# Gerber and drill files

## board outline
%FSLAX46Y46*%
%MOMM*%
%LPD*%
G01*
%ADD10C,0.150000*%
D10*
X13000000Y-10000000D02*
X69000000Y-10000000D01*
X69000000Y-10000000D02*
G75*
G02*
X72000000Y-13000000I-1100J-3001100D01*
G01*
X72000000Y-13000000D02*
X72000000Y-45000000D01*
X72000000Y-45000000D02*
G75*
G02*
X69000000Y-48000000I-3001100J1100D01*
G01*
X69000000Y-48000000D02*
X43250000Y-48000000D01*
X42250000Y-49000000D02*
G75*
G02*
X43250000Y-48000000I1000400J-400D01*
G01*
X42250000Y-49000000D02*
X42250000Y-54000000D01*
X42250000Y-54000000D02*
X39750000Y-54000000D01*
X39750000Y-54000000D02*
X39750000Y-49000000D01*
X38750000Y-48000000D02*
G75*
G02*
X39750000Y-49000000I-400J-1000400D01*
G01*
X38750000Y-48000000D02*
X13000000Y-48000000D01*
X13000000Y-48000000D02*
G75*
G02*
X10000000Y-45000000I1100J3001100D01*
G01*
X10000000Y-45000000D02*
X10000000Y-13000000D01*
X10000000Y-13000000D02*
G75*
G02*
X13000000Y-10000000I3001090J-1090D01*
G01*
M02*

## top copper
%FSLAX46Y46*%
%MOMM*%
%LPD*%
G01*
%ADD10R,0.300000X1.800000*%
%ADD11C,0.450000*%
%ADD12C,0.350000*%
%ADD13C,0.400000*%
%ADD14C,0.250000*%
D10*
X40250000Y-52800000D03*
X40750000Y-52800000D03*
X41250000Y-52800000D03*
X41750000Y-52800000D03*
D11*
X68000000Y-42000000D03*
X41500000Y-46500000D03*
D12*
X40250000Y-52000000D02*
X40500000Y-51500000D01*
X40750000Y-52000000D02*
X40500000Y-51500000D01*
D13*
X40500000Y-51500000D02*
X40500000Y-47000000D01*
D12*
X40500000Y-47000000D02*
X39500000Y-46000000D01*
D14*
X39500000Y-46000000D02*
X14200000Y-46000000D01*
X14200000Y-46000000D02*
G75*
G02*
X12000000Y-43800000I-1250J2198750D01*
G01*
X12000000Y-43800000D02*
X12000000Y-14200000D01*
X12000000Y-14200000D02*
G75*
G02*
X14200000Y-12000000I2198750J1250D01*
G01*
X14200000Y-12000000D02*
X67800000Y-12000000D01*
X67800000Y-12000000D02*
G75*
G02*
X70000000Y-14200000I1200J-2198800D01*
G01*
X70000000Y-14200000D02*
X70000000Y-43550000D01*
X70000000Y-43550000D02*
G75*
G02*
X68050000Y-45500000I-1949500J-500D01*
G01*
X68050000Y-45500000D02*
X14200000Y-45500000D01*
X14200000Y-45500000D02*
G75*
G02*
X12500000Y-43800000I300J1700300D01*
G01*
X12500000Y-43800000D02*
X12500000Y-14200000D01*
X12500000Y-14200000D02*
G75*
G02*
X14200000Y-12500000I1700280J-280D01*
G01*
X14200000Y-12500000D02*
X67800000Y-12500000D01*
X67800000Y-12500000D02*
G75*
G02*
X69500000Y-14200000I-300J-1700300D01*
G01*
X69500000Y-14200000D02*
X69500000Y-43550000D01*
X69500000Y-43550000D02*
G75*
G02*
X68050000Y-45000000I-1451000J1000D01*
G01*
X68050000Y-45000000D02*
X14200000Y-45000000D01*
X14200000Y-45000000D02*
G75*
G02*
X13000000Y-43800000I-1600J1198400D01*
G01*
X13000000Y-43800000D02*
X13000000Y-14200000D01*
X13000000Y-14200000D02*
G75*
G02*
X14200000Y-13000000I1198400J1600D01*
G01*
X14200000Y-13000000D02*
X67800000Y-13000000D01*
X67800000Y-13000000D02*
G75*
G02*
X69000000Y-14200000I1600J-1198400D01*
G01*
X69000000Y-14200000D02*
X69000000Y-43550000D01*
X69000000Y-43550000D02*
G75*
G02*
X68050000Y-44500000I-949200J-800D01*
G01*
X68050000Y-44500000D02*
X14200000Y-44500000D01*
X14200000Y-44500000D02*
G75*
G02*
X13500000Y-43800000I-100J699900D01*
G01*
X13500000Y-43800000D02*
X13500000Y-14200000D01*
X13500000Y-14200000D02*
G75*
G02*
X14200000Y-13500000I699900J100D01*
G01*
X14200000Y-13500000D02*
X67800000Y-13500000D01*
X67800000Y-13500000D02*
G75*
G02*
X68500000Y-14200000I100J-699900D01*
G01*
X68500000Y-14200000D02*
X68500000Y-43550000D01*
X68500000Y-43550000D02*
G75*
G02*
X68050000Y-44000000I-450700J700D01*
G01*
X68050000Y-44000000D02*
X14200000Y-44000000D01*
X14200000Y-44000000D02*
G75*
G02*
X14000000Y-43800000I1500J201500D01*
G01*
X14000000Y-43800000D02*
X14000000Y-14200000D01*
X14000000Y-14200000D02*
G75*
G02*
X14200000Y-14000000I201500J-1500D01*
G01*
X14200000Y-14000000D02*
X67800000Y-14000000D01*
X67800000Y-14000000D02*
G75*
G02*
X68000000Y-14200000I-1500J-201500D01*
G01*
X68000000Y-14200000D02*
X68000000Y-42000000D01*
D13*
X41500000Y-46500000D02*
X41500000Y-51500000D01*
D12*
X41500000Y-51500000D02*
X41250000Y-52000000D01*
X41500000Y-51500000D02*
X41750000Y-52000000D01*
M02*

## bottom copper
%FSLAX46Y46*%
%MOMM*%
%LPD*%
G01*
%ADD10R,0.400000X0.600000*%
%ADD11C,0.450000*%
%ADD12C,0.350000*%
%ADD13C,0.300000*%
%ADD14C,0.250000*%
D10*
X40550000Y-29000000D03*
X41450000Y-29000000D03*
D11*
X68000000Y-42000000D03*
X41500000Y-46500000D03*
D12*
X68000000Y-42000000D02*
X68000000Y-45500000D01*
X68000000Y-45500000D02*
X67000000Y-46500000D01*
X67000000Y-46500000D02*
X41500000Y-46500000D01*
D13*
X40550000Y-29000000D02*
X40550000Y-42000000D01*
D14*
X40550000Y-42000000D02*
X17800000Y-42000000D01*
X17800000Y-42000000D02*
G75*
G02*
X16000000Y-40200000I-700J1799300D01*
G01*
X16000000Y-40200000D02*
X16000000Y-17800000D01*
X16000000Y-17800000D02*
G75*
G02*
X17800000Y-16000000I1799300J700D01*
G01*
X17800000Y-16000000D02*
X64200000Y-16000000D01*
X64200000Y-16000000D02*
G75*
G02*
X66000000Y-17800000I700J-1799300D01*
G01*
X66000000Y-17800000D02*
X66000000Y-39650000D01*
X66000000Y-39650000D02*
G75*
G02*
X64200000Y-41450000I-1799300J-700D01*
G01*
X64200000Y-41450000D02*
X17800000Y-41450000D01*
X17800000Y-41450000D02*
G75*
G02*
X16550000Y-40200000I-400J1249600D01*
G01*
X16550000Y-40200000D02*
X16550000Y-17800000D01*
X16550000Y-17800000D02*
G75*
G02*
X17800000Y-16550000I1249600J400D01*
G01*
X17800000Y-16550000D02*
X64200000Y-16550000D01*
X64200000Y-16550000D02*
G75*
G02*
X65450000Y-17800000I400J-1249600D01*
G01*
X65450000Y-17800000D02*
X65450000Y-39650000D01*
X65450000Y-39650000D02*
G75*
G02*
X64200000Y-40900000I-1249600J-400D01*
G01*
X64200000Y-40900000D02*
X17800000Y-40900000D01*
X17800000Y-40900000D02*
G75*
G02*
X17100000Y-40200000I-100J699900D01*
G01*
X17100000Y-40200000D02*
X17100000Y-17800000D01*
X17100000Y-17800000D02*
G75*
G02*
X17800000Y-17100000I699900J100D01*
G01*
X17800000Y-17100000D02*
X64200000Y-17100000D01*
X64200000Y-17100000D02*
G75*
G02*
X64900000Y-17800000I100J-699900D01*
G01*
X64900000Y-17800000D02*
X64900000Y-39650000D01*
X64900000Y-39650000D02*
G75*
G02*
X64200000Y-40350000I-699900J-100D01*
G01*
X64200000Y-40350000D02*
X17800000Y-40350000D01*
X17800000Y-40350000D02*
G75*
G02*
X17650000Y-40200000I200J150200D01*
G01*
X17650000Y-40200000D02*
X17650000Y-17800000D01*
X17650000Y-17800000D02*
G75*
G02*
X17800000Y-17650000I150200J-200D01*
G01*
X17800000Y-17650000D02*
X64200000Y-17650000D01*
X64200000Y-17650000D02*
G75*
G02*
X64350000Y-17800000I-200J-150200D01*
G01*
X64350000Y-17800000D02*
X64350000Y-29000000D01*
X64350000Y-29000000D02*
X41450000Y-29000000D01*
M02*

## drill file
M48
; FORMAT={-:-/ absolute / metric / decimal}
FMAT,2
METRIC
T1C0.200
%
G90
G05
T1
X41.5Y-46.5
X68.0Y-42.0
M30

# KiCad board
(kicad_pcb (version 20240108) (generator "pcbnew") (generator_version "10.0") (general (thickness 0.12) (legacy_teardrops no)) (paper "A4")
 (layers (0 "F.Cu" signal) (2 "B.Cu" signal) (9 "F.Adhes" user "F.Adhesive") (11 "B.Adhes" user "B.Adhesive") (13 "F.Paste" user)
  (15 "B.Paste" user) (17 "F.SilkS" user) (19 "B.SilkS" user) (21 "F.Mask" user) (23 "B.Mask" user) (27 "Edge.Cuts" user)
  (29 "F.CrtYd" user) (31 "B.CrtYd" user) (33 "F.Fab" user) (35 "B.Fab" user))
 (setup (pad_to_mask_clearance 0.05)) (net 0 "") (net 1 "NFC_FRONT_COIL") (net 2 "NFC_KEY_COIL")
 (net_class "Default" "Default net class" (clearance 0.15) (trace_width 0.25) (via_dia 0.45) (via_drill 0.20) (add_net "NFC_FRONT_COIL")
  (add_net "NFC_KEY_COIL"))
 (gr_line (start 13.000 10.000) (end 69.000 10.000) (stroke (width 0.15) (type solid)) (layer "Edge.Cuts"))
 (gr_arc (start 69.000 10.000) (mid 71.121 10.879) (end 72.000 13.000) (stroke (width 0.15) (type solid)) (layer "Edge.Cuts"))
 (gr_line (start 72.000 13.000) (end 72.000 45.000) (stroke (width 0.15) (type solid)) (layer "Edge.Cuts"))
 (gr_arc (start 72.000 45.000) (mid 71.121 47.121) (end 69.000 48.000) (stroke (width 0.15) (type solid)) (layer "Edge.Cuts"))
 (gr_line (start 69.000 48.000) (end 43.250 48.000) (stroke (width 0.15) (type solid)) (layer "Edge.Cuts"))
 (gr_arc (start 43.250 48.000) (mid 42.543 48.293) (end 42.250 49.000) (stroke (width 0.15) (type solid)) (layer "Edge.Cuts"))
 (gr_line (start 42.250 49.000) (end 42.250 54.000) (stroke (width 0.15) (type solid)) (layer "Edge.Cuts"))
 (gr_line (start 42.250 54.000) (end 39.750 54.000) (stroke (width 0.15) (type solid)) (layer "Edge.Cuts"))
 (gr_line (start 39.750 54.000) (end 39.750 49.000) (stroke (width 0.15) (type solid)) (layer "Edge.Cuts"))
 (gr_arc (start 39.750 49.000) (mid 39.457 48.293) (end 38.750 48.000) (stroke (width 0.15) (type solid)) (layer "Edge.Cuts"))
 (gr_line (start 38.750 48.000) (end 13.000 48.000) (stroke (width 0.15) (type solid)) (layer "Edge.Cuts"))
 (gr_arc (start 13.000 48.000) (mid 10.879 47.121) (end 10.000 45.000) (stroke (width 0.15) (type solid)) (layer "Edge.Cuts"))
 (gr_line (start 10.000 45.000) (end 10.000 13.000) (stroke (width 0.15) (type solid)) (layer "Edge.Cuts"))
 (gr_arc (start 10.000 13.000) (mid 10.879 10.879) (end 13.000 10.000) (stroke (width 0.15) (type solid)) (layer "Edge.Cuts"))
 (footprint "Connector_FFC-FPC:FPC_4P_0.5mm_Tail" (layer "F.Cu") (at 41.0 52.8 0)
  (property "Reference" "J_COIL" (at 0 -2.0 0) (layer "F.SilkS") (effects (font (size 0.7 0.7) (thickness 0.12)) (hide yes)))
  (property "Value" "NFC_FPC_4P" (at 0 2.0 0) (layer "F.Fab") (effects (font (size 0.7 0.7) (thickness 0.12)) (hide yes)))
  (pad "1" smd rect (at -0.750 0.000) (size 0.300 1.800) (layers "F.Cu" "F.Mask") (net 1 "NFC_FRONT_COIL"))
  (pad "2" smd rect (at -0.250 0.000) (size 0.300 1.800) (layers "F.Cu" "F.Mask") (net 1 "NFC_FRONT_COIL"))
  (pad "3" smd rect (at 0.250 0.000) (size 0.300 1.800) (layers "F.Cu" "F.Mask") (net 1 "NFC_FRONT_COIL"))
  (pad "4" smd rect (at 0.750 0.000) (size 0.300 1.800) (layers "F.Cu" "F.Mask") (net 1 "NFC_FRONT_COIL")))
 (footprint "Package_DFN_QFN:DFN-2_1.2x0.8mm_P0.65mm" (layer "B.Cu") (at 41.0 29.0 0)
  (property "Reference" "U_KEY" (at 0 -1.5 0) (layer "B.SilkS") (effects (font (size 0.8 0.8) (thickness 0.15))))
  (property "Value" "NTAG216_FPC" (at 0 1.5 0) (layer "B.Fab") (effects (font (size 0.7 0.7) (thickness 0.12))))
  (pad "1" smd rect (at -0.45 0.0) (size 0.40 0.60) (layers "B.Cu" "B.Mask" "B.Paste") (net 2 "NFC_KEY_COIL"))
  (pad "2" smd rect (at 0.45 0.0) (size 0.40 0.60) (layers "B.Cu" "B.Mask" "B.Paste") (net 2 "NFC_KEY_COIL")))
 (segment (start 40.250 52.000) (end 40.500 51.500) (width 0.350) (layer "F.Cu") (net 1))
 (segment (start 40.750 52.000) (end 40.500 51.500) (width 0.350) (layer "F.Cu") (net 1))
 (segment (start 40.500 51.500) (end 40.500 47.000) (width 0.400) (layer "F.Cu") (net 1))
 (arc (start 40.500 47.000) (mid 40.207 46.707) (end 39.500 46.000) (width 0.350) (layer "F.Cu") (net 1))
 (segment (start 39.500 46.000) (end 14.200 46.000) (width 0.250) (layer "F.Cu") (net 1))
 (arc (start 14.200 46.000) (mid 12.644 45.356) (end 12.000 43.800) (width 0.250) (layer "F.Cu") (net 1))
 (segment (start 12.000 43.800) (end 12.000 14.200) (width 0.250) (layer "F.Cu") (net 1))
 (arc (start 12.000 14.200) (mid 12.644 12.644) (end 14.200 12.000) (width 0.250) (layer "F.Cu") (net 1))
 (segment (start 14.200 12.000) (end 67.800 12.000) (width 0.250) (layer "F.Cu") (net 1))
 (arc (start 67.800 12.000) (mid 69.356 12.644) (end 70.000 14.200) (width 0.250) (layer "F.Cu") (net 1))
 (segment (start 70.000 14.200) (end 70.000 43.550) (width 0.250) (layer "F.Cu") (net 1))
 (arc (start 70.000 43.550) (mid 69.429 44.929) (end 68.050 45.500) (width 0.250) (layer "F.Cu") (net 1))
 (segment (start 68.050 45.500) (end 14.200 45.500) (width 0.250) (layer "F.Cu") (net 1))
 (arc (start 14.200 45.500) (mid 12.998 45.002) (end 12.500 43.800) (width 0.250) (layer "F.Cu") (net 1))
 (segment (start 12.500 43.800) (end 12.500 14.200) (width 0.250) (layer "F.Cu") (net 1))
 (arc (start 12.500 14.200) (mid 12.998 12.998) (end 14.200 12.500) (width 0.250) (layer "F.Cu") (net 1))
 (segment (start 14.200 12.500) (end 67.800 12.500) (width 0.250) (layer "F.Cu") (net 1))
 (arc (start 67.800 12.500) (mid 69.002 12.998) (end 69.500 14.200) (width 0.250) (layer "F.Cu") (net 1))
 (segment (start 69.500 14.200) (end 69.500 43.550) (width 0.250) (layer "F.Cu") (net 1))
 (arc (start 69.500 43.550) (mid 69.075 44.575) (end 68.050 45.000) (width 0.250) (layer "F.Cu") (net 1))
 (segment (start 68.050 45.000) (end 14.200 45.000) (width 0.250) (layer "F.Cu") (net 1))
 (arc (start 14.200 45.000) (mid 13.351 44.649) (end 13.000 43.800) (width 0.250) (layer "F.Cu") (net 1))
 (segment (start 13.000 43.800) (end 13.000 14.200) (width 0.250) (layer "F.Cu") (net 1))
 (arc (start 13.000 14.200) (mid 13.351 13.351) (end 14.200 13.000) (width 0.250) (layer "F.Cu") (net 1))
 (segment (start 14.200 13.000) (end 67.800 13.000) (width 0.250) (layer "F.Cu") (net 1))
 (arc (start 67.800 13.000) (mid 68.649 13.351) (end 69.000 14.200) (width 0.250) (layer "F.Cu") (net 1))
 (segment (start 69.000 14.200) (end 69.000 43.550) (width 0.250) (layer "F.Cu") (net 1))
 (arc (start 69.000 43.550) (mid 68.722 44.222) (end 68.050 44.500) (width 0.250) (layer "F.Cu") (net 1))
 (segment (start 68.050 44.500) (end 14.200 44.500) (width 0.250) (layer "F.Cu") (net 1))
 (arc (start 14.200 44.500) (mid 13.705 44.295) (end 13.500 43.800) (width 0.250) (layer "F.Cu") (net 1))
 (segment (start 13.500 43.800) (end 13.500 14.200) (width 0.250) (layer "F.Cu") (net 1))
 (arc (start 13.500 14.200) (mid 13.705 13.705) (end 14.200 13.500) (width 0.250) (layer "F.Cu") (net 1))
 (segment (start 14.200 13.500) (end 67.800 13.500) (width 0.250) (layer "F.Cu") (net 1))
 (arc (start 67.800 13.500) (mid 68.295 13.705) (end 68.500 14.200) (width 0.250) (layer "F.Cu") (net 1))
 (segment (start 68.500 14.200) (end 68.500 43.550) (width 0.250) (layer "F.Cu") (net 1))
 (arc (start 68.500 43.550) (mid 68.368 43.868) (end 68.050 44.000) (width 0.250) (layer "F.Cu") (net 1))
 (segment (start 68.050 44.000) (end 14.200 44.000) (width 0.250) (layer "F.Cu") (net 1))
 (arc (start 14.200 44.000) (mid 14.059 43.941) (end 14.000 43.800) (width 0.250) (layer "F.Cu") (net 1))
 (segment (start 14.000 43.800) (end 14.000 14.200) (width 0.250) (layer "F.Cu") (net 1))
 (arc (start 14.000 14.200) (mid 14.059 14.059) (end 14.200 14.000) (width 0.250) (layer "F.Cu") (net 1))
 (segment (start 14.200 14.000) (end 67.800 14.000) (width 0.250) (layer "F.Cu") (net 1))
 (arc (start 67.800 14.000) (mid 67.941 14.059) (end 68.000 14.200) (width 0.250) (layer "F.Cu") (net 1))
 (segment (start 68.000 14.200) (end 68.000 42.000) (width 0.250) (layer "F.Cu") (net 1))
 (via (at 68.000 42.000) (size 0.450) (drill 0.200) (layers "F.Cu" "B.Cu") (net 1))
 (via (at 41.500 46.500) (size 0.450) (drill 0.200) (layers "F.Cu" "B.Cu") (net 1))
 (segment (start 68.000 42.000) (end 68.000 45.500) (width 0.350) (layer "B.Cu") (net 1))
 (segment (start 68.000 45.500) (end 67.000 46.500) (width 0.350) (layer "B.Cu") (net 1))
 (segment (start 67.000 46.500) (end 41.500 46.500) (width 0.350) (layer "B.Cu") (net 1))
 (segment (start 41.500 46.500) (end 41.500 51.500) (width 0.400) (layer "F.Cu") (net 1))
 (segment (start 41.500 51.500) (end 41.250 52.000) (width 0.350) (layer "F.Cu") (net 1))
 (segment (start 41.500 51.500) (end 41.750 52.000) (width 0.350) (layer "F.Cu") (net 1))
 (segment (start 40.550 29.000) (end 40.550 42.000) (width 0.300) (layer "B.Cu") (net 2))
 (segment (start 40.550 42.000) (end 17.800 42.000) (width 0.250) (layer "B.Cu") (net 2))
 (arc (start 17.800 42.000) (mid 16.527 41.473) (end 16.000 40.200) (width 0.250) (layer "B.Cu") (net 2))
 (segment (start 16.000 40.200) (end 16.000 17.800) (width 0.250) (layer "B.Cu") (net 2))
 (arc (start 16.000 17.800) (mid 16.527 16.527) (end 17.800 16.000) (width 0.250) (layer "B.Cu") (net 2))
 (segment (start 17.800 16.000) (end 64.200 16.000) (width 0.250) (layer "B.Cu") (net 2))
 (arc (start 64.200 16.000) (mid 65.473 16.527) (end 66.000 17.800) (width 0.250) (layer "B.Cu") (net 2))
 (segment (start 66.000 17.800) (end 66.000 39.650) (width 0.250) (layer "B.Cu") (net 2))
 (arc (start 66.000 39.650) (mid 65.473 40.923) (end 64.200 41.450) (width 0.250) (layer "B.Cu") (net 2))
 (segment (start 64.200 41.450) (end 17.800 41.450) (width 0.250) (layer "B.Cu") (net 2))
 (arc (start 17.800 41.450) (mid 16.916 41.084) (end 16.550 40.200) (width 0.250) (layer "B.Cu") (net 2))
 (segment (start 16.550 40.200) (end 16.550 17.800) (width 0.250) (layer "B.Cu") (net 2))
 (arc (start 16.550 17.800) (mid 16.916 16.916) (end 17.800 16.550) (width 0.250) (layer "B.Cu") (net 2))
 (segment (start 17.800 16.550) (end 64.200 16.550) (width 0.250) (layer "B.Cu") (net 2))
 (arc (start 64.200 16.550) (mid 65.084 16.916) (end 65.450 17.800) (width 0.250) (layer "B.Cu") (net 2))
 (segment (start 65.450 17.800) (end 65.450 39.650) (width 0.250) (layer "B.Cu") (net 2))
 (arc (start 65.450 39.650) (mid 65.084 40.534) (end 64.200 40.900) (width 0.250) (layer "B.Cu") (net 2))
 (segment (start 64.200 40.900) (end 17.800 40.900) (width 0.250) (layer "B.Cu") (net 2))
 (arc (start 17.800 40.900) (mid 17.305 40.695) (end 17.100 40.200) (width 0.250) (layer "B.Cu") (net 2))
 (segment (start 17.100 40.200) (end 17.100 17.800) (width 0.250) (layer "B.Cu") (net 2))
 (arc (start 17.100 17.800) (mid 17.305 17.305) (end 17.800 17.100) (width 0.250) (layer "B.Cu") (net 2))
 (segment (start 17.800 17.100) (end 64.200 17.100) (width 0.250) (layer "B.Cu") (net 2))
 (arc (start 64.200 17.100) (mid 64.695 17.305) (end 64.900 17.800) (width 0.250) (layer "B.Cu") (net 2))
 (segment (start 64.900 17.800) (end 64.900 39.650) (width 0.250) (layer "B.Cu") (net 2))
 (arc (start 64.900 39.650) (mid 64.695 40.145) (end 64.200 40.350) (width 0.250) (layer "B.Cu") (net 2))
 (segment (start 64.200 40.350) (end 17.800 40.350) (width 0.250) (layer "B.Cu") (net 2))
 (arc (start 17.800 40.350) (mid 17.694 40.306) (end 17.650 40.200) (width 0.250) (layer "B.Cu") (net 2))
 (segment (start 17.650 40.200) (end 17.650 17.800) (width 0.250) (layer "B.Cu") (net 2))
 (arc (start 17.650 17.800) (mid 17.694 17.694) (end 17.800 17.650) (width 0.250) (layer "B.Cu") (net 2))
 (segment (start 17.800 17.650) (end 64.200 17.650) (width 0.250) (layer "B.Cu") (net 2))
 (arc (start 64.200 17.650) (mid 64.306 17.694) (end 64.350 17.800) (width 0.250) (layer "B.Cu") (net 2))
 (segment (start 64.350 17.800) (end 64.350 29.000) (width 0.250) (layer "B.Cu") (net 2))
 (segment (start 64.350 29.000) (end 41.450 29.000) (width 0.250) (layer "B.Cu") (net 2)))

